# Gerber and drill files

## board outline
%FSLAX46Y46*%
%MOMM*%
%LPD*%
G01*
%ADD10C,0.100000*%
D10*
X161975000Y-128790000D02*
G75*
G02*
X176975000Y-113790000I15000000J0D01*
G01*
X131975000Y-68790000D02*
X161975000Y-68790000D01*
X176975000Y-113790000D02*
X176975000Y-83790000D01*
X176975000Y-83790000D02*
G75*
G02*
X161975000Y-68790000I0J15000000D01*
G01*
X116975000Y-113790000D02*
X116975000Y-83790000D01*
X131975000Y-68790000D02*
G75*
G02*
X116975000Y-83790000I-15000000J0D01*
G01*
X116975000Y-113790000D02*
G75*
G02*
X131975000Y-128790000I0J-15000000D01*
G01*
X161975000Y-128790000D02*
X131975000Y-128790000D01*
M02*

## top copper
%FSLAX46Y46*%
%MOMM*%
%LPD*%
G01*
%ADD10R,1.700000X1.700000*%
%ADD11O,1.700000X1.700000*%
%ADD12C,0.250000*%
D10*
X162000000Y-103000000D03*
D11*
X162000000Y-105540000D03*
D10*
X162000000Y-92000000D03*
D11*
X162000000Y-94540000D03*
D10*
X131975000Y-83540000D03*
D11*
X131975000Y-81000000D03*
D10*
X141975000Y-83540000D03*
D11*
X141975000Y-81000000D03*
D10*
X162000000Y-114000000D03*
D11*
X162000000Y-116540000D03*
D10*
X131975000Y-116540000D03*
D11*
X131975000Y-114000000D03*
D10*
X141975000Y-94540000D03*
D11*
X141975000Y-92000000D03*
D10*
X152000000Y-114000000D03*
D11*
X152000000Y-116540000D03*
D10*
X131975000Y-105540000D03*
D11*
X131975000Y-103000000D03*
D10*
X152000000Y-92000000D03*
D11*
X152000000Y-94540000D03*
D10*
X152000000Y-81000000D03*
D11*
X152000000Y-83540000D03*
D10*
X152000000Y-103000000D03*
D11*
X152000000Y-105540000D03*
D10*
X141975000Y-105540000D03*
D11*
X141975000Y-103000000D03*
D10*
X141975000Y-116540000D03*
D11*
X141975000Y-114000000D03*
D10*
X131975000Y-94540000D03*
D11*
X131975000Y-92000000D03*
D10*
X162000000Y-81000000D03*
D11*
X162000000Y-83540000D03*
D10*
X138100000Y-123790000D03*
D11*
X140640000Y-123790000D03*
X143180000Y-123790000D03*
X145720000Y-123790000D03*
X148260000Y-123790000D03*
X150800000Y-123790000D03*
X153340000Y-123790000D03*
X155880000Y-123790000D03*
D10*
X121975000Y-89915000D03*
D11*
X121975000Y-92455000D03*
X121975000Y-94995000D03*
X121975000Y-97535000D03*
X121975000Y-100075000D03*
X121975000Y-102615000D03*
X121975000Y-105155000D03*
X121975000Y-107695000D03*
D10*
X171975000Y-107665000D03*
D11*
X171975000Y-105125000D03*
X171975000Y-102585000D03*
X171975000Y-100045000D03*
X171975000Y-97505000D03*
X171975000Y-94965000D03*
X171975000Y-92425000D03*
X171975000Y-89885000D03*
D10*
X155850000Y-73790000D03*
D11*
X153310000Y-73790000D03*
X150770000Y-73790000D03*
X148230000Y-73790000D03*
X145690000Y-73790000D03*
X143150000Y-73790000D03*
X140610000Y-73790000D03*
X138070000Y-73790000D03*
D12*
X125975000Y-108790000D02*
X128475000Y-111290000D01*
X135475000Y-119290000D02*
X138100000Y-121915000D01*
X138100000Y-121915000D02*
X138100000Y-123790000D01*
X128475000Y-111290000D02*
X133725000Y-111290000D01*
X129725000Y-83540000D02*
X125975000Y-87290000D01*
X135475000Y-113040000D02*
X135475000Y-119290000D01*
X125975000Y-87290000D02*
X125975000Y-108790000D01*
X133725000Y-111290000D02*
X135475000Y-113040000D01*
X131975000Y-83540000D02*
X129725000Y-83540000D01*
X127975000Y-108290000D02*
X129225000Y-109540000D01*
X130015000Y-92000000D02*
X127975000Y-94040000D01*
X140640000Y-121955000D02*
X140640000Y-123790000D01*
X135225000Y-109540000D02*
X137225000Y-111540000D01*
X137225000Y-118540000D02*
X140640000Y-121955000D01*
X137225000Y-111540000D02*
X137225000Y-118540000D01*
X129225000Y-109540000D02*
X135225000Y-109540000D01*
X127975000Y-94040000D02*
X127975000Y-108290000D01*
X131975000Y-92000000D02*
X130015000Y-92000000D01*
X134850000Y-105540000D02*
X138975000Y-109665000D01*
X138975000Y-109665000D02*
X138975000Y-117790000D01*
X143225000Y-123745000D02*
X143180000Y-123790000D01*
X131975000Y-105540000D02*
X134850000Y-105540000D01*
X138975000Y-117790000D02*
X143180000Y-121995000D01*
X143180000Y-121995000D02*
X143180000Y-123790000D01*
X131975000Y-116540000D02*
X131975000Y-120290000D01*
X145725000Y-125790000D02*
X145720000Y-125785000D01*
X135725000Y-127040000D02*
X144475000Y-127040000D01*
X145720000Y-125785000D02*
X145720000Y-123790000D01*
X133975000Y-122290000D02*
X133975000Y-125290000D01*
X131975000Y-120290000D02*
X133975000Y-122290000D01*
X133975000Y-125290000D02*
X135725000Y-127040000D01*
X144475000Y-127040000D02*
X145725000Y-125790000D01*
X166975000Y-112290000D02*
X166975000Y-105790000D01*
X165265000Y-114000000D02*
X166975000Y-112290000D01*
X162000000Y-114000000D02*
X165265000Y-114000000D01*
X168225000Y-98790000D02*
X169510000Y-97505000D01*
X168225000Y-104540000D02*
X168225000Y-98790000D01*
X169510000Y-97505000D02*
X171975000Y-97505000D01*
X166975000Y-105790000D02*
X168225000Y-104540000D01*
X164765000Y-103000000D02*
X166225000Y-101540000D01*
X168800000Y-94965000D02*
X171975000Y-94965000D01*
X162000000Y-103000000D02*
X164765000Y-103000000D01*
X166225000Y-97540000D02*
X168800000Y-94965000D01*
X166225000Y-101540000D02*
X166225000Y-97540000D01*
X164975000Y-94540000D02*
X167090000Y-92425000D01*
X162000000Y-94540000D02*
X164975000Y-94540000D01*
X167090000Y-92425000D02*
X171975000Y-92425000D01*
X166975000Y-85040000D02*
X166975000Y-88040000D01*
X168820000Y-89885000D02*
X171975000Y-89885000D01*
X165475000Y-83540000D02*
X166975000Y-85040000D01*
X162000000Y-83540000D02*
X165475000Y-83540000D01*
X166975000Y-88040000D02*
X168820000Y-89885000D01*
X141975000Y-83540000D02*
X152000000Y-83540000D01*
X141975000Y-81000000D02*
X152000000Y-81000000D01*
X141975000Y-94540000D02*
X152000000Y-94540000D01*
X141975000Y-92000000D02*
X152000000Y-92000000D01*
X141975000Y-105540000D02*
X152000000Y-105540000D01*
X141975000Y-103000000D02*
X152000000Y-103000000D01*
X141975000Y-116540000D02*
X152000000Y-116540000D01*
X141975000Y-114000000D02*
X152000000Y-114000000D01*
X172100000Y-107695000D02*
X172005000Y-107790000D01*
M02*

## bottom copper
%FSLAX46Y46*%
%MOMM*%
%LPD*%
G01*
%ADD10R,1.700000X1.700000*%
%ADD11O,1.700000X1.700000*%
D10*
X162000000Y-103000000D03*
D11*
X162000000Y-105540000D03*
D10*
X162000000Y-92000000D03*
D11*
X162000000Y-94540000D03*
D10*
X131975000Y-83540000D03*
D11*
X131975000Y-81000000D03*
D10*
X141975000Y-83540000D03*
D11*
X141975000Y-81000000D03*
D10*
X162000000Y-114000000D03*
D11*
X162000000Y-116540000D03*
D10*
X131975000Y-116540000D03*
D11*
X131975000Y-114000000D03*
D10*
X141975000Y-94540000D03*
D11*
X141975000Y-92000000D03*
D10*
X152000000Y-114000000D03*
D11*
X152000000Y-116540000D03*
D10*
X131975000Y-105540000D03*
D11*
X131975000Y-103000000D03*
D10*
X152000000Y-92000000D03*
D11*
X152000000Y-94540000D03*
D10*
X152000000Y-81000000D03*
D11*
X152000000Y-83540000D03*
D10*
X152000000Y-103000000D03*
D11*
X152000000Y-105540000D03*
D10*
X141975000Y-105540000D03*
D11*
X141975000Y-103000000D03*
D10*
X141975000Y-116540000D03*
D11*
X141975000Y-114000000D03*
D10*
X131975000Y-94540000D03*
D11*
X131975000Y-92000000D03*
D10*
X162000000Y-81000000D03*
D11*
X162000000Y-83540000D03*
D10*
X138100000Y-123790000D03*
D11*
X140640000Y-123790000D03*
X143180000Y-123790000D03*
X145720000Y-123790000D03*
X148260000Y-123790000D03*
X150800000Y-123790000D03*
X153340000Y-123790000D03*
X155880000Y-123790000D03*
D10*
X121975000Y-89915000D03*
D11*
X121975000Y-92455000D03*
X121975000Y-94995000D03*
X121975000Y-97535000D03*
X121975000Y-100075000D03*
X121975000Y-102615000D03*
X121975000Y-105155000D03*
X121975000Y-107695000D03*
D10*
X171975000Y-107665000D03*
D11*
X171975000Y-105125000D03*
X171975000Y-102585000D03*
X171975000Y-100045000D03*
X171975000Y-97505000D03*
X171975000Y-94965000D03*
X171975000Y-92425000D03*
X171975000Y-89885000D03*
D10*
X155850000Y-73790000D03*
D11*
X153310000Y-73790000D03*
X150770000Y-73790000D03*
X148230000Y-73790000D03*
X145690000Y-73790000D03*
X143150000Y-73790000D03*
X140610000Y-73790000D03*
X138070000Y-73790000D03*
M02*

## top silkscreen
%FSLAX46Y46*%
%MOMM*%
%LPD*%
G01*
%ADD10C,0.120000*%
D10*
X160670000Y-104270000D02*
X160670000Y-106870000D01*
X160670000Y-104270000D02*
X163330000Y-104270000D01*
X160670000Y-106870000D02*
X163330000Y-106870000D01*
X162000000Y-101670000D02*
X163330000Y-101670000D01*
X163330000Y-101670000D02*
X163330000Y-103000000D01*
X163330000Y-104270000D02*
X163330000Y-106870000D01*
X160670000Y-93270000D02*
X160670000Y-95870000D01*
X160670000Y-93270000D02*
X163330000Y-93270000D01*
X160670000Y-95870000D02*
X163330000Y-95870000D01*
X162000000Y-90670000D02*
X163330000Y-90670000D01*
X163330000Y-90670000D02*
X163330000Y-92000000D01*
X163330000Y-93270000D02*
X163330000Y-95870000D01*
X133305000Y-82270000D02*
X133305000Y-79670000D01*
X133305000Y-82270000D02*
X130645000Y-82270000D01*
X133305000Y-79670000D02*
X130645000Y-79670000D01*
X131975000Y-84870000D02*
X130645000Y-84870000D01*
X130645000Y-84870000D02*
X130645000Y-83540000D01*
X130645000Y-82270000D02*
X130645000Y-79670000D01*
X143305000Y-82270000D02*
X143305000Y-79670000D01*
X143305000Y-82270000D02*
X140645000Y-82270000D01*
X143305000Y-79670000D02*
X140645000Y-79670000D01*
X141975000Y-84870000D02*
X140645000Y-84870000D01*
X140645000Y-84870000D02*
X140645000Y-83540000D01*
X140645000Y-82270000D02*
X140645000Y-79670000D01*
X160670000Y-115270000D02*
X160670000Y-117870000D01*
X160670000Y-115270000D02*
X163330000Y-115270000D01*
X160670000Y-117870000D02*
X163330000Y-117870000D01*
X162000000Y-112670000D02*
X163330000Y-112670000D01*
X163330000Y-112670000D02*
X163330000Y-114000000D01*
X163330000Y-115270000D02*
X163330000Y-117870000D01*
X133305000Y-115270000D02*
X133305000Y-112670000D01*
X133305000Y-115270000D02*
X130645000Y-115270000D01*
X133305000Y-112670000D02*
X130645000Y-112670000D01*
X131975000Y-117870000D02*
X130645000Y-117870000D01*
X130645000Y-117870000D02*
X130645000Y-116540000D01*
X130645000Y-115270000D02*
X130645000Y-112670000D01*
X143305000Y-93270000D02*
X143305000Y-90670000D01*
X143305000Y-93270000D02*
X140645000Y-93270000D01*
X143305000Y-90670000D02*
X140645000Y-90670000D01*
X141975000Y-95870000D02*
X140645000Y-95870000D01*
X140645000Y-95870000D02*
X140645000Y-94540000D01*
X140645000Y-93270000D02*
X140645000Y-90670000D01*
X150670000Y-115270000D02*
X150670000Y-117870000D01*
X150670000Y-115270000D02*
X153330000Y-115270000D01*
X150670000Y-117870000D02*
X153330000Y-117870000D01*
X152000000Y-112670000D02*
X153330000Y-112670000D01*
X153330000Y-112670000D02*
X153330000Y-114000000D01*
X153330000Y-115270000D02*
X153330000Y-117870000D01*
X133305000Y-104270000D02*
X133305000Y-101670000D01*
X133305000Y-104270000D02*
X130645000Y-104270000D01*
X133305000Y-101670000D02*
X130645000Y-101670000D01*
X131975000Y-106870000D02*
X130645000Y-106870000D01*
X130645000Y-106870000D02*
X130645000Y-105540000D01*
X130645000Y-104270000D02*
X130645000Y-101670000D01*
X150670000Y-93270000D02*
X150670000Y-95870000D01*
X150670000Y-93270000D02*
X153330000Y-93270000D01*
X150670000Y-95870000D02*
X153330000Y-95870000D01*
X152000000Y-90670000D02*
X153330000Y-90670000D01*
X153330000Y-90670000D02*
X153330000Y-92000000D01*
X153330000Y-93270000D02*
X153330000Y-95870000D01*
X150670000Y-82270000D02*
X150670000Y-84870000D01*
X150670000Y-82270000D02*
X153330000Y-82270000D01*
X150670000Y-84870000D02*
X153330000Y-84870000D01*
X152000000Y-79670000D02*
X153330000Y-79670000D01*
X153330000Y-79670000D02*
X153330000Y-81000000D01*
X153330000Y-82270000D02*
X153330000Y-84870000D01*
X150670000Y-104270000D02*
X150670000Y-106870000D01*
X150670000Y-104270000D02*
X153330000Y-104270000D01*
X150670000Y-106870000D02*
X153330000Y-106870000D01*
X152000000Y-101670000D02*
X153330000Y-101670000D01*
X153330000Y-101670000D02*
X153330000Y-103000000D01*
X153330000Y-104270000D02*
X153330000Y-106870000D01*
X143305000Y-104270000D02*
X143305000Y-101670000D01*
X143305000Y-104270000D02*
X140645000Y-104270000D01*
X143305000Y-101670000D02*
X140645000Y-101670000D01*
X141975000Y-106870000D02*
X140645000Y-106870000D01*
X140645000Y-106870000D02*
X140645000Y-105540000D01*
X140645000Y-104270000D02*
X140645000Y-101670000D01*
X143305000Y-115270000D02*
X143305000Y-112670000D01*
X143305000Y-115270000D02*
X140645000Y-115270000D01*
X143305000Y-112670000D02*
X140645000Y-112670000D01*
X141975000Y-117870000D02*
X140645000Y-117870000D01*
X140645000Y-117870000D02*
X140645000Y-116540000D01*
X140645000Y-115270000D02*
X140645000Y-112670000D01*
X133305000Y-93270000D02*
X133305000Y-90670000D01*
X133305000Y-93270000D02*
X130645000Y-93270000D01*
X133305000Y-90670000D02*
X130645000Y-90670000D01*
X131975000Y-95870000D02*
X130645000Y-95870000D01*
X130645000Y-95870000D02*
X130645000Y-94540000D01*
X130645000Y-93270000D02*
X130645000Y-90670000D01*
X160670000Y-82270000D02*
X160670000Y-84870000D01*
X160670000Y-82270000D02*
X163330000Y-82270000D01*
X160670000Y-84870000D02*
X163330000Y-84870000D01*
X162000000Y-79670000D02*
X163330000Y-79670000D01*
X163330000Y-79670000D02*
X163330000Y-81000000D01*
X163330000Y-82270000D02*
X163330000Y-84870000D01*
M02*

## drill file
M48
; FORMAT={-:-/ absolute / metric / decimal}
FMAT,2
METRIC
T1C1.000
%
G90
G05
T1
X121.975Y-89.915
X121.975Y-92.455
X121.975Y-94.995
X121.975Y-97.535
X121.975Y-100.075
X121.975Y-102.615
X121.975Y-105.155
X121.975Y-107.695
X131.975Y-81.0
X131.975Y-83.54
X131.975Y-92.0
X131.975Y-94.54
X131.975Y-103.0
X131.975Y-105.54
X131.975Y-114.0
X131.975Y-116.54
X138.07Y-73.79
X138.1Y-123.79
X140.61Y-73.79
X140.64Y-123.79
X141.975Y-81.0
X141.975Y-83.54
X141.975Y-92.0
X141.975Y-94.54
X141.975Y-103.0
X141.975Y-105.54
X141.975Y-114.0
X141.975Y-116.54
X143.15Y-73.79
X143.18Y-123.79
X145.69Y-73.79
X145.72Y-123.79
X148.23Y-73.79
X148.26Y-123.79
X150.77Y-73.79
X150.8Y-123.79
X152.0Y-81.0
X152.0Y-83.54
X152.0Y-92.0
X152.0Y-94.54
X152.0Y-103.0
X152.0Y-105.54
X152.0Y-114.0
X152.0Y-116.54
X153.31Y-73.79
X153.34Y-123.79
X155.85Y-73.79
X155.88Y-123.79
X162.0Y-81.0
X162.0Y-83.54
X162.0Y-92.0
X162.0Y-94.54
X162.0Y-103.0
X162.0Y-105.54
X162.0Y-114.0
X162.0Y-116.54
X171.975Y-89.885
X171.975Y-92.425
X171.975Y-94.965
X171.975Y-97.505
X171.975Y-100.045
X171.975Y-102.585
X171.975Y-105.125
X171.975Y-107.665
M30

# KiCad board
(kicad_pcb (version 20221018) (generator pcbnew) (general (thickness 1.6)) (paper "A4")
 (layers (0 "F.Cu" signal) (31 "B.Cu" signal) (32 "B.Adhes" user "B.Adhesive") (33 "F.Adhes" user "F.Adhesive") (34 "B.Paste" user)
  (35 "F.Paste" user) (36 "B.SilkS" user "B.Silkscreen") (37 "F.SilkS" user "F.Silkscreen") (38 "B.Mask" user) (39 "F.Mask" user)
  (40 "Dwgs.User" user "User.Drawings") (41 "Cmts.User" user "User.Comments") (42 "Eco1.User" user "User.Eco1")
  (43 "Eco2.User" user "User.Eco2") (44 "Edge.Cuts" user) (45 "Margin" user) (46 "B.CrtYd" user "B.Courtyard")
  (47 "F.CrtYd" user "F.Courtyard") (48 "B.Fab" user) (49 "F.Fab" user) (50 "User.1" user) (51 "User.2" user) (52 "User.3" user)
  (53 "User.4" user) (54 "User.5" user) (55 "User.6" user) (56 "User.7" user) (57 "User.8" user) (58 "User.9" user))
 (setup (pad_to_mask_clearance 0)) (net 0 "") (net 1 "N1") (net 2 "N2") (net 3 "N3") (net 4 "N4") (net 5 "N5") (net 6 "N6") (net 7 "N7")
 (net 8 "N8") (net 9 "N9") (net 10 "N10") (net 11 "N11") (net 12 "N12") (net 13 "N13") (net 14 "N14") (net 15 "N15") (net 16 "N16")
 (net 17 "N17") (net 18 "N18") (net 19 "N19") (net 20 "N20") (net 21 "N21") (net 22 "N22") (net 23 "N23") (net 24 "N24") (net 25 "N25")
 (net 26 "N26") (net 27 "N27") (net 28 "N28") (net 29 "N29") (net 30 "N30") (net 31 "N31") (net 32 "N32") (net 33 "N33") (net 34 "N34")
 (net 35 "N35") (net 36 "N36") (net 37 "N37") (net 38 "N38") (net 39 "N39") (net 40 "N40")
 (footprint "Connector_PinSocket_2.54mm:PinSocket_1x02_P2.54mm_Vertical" (layer "F.Cu") (at 162 103)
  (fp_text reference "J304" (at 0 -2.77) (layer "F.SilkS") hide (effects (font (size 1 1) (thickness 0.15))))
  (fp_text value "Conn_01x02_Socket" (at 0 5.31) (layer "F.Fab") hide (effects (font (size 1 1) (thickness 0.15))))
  (fp_line (start -1.33 1.27) (end -1.33 3.87) (stroke (width 0.12) (type solid)) (layer "F.SilkS"))
  (fp_line (start -1.33 1.27) (end 1.33 1.27) (stroke (width 0.12) (type solid)) (layer "F.SilkS"))
  (fp_line (start -1.33 3.87) (end 1.33 3.87) (stroke (width 0.12) (type solid)) (layer "F.SilkS"))
  (fp_line (start 0 -1.33) (end 1.33 -1.33) (stroke (width 0.12) (type solid)) (layer "F.SilkS"))
  (fp_line (start 1.33 -1.33) (end 1.33 0) (stroke (width 0.12) (type solid)) (layer "F.SilkS"))
  (fp_line (start 1.33 1.27) (end 1.33 3.87) (stroke (width 0.12) (type solid)) (layer "F.SilkS"))
  (pad "1" thru_hole rect (at 0 0) (size 1.7 1.7) (drill 1) (layers "*.Cu" "*.Mask") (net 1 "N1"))
  (pad "2" thru_hole oval (at 0 2.54) (size 1.7 1.7) (drill 1) (layers "*.Cu" "*.Mask") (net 1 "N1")))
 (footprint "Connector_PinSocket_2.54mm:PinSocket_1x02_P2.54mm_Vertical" (layer "F.Cu") (at 162 92)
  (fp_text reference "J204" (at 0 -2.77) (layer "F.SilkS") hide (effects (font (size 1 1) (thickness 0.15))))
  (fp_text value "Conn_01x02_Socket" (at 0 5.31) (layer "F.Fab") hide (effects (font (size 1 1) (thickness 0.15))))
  (fp_line (start -1.33 1.27) (end -1.33 3.87) (stroke (width 0.12) (type solid)) (layer "F.SilkS"))
  (fp_line (start -1.33 1.27) (end 1.33 1.27) (stroke (width 0.12) (type solid)) (layer "F.SilkS"))
  (fp_line (start -1.33 3.87) (end 1.33 3.87) (stroke (width 0.12) (type solid)) (layer "F.SilkS"))
  (fp_line (start 0 -1.33) (end 1.33 -1.33) (stroke (width 0.12) (type solid)) (layer "F.SilkS"))
  (fp_line (start 1.33 -1.33) (end 1.33 0) (stroke (width 0.12) (type solid)) (layer "F.SilkS"))
  (fp_line (start 1.33 1.27) (end 1.33 3.87) (stroke (width 0.12) (type solid)) (layer "F.SilkS"))
  (pad "1" thru_hole rect (at 0 0) (size 1.7 1.7) (drill 1) (layers "*.Cu" "*.Mask") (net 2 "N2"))
  (pad "2" thru_hole oval (at 0 2.54) (size 1.7 1.7) (drill 1) (layers "*.Cu" "*.Mask") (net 2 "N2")))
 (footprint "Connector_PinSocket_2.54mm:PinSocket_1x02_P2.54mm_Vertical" (layer "F.Cu") (at 131.975 83.54 180)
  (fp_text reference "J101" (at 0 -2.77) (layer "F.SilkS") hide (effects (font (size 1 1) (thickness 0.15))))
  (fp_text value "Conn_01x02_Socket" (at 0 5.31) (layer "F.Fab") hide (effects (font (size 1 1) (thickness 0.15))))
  (fp_line (start -1.33 1.27) (end -1.33 3.87) (stroke (width 0.12) (type solid)) (layer "F.SilkS"))
  (fp_line (start -1.33 1.27) (end 1.33 1.27) (stroke (width 0.12) (type solid)) (layer "F.SilkS"))
  (fp_line (start -1.33 3.87) (end 1.33 3.87) (stroke (width 0.12) (type solid)) (layer "F.SilkS"))
  (fp_line (start 0 -1.33) (end 1.33 -1.33) (stroke (width 0.12) (type solid)) (layer "F.SilkS"))
  (fp_line (start 1.33 -1.33) (end 1.33 0) (stroke (width 0.12) (type solid)) (layer "F.SilkS"))
  (fp_line (start 1.33 1.27) (end 1.33 3.87) (stroke (width 0.12) (type solid)) (layer "F.SilkS"))
  (pad "1" thru_hole rect (at 0 0 180) (size 1.7 1.7) (drill 1) (layers "*.Cu" "*.Mask") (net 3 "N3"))
  (pad "2" thru_hole oval (at 0 2.54 180) (size 1.7 1.7) (drill 1) (layers "*.Cu" "*.Mask") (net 3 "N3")))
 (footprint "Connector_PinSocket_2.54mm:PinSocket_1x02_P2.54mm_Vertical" (layer "F.Cu") (at 141.975 83.54 180)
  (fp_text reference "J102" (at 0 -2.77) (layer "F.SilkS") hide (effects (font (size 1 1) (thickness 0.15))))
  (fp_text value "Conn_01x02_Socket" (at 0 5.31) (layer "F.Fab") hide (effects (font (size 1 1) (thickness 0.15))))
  (fp_line (start -1.33 1.27) (end -1.33 3.87) (stroke (width 0.12) (type solid)) (layer "F.SilkS"))
  (fp_line (start -1.33 1.27) (end 1.33 1.27) (stroke (width 0.12) (type solid)) (layer "F.SilkS"))
  (fp_line (start -1.33 3.87) (end 1.33 3.87) (stroke (width 0.12) (type solid)) (layer "F.SilkS"))
  (fp_line (start 0 -1.33) (end 1.33 -1.33) (stroke (width 0.12) (type solid)) (layer "F.SilkS"))
  (fp_line (start 1.33 -1.33) (end 1.33 0) (stroke (width 0.12) (type solid)) (layer "F.SilkS"))
  (fp_line (start 1.33 1.27) (end 1.33 3.87) (stroke (width 0.12) (type solid)) (layer "F.SilkS"))
  (pad "1" thru_hole rect (at 0 0 180) (size 1.7 1.7) (drill 1) (layers "*.Cu" "*.Mask") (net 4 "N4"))
  (pad "2" thru_hole oval (at 0 2.54 180) (size 1.7 1.7) (drill 1) (layers "*.Cu" "*.Mask") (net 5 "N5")))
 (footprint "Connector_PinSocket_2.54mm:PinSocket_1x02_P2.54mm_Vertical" (layer "F.Cu") (at 162 114)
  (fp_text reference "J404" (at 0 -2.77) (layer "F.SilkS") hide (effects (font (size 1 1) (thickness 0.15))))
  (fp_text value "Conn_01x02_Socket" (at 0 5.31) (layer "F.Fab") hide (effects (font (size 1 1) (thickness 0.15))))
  (fp_line (start -1.33 1.27) (end -1.33 3.87) (stroke (width 0.12) (type solid)) (layer "F.SilkS"))
  (fp_line (start -1.33 1.27) (end 1.33 1.27) (stroke (width 0.12) (type solid)) (layer "F.SilkS"))
  (fp_line (start -1.33 3.87) (end 1.33 3.87) (stroke (width 0.12) (type solid)) (layer "F.SilkS"))
  (fp_line (start 0 -1.33) (end 1.33 -1.33) (stroke (width 0.12) (type solid)) (layer "F.SilkS"))
  (fp_line (start 1.33 -1.33) (end 1.33 0) (stroke (width 0.12) (type solid)) (layer "F.SilkS"))
  (fp_line (start 1.33 1.27) (end 1.33 3.87) (stroke (width 0.12) (type solid)) (layer "F.SilkS"))
  (pad "1" thru_hole rect (at 0 0) (size 1.7 1.7) (drill 1) (layers "*.Cu" "*.Mask") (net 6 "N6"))
  (pad "2" thru_hole oval (at 0 2.54) (size 1.7 1.7) (drill 1) (layers "*.Cu" "*.Mask") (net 6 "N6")))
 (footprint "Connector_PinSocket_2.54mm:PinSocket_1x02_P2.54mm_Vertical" (layer "F.Cu") (at 131.975 116.54 180)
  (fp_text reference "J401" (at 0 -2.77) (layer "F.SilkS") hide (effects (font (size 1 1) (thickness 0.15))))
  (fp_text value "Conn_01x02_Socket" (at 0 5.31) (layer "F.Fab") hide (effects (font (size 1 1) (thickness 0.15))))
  (fp_line (start -1.33 1.27) (end -1.33 3.87) (stroke (width 0.12) (type solid)) (layer "F.SilkS"))
  (fp_line (start -1.33 1.27) (end 1.33 1.27) (stroke (width 0.12) (type solid)) (layer "F.SilkS"))
  (fp_line (start -1.33 3.87) (end 1.33 3.87) (stroke (width 0.12) (type solid)) (layer "F.SilkS"))
  (fp_line (start 0 -1.33) (end 1.33 -1.33) (stroke (width 0.12) (type solid)) (layer "F.SilkS"))
  (fp_line (start 1.33 -1.33) (end 1.33 0) (stroke (width 0.12) (type solid)) (layer "F.SilkS"))
  (fp_line (start 1.33 1.27) (end 1.33 3.87) (stroke (width 0.12) (type solid)) (layer "F.SilkS"))
  (pad "1" thru_hole rect (at 0 0 180) (size 1.7 1.7) (drill 1) (layers "*.Cu" "*.Mask") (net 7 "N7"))
  (pad "2" thru_hole oval (at 0 2.54 180) (size 1.7 1.7) (drill 1) (layers "*.Cu" "*.Mask") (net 7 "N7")))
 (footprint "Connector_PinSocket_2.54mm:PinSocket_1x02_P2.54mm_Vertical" (layer "F.Cu") (at 141.975 94.54 180)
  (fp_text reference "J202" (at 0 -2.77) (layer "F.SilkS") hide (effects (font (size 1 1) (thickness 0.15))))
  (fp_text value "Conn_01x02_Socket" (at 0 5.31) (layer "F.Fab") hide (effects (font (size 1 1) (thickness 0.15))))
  (fp_line (start -1.33 1.27) (end -1.33 3.87) (stroke (width 0.12) (type solid)) (layer "F.SilkS"))
  (fp_line (start -1.33 1.27) (end 1.33 1.27) (stroke (width 0.12) (type solid)) (layer "F.SilkS"))
  (fp_line (start -1.33 3.87) (end 1.33 3.87) (stroke (width 0.12) (type solid)) (layer "F.SilkS"))
  (fp_line (start 0 -1.33) (end 1.33 -1.33) (stroke (width 0.12) (type solid)) (layer "F.SilkS"))
  (fp_line (start 1.33 -1.33) (end 1.33 0) (stroke (width 0.12) (type solid)) (layer "F.SilkS"))
  (fp_line (start 1.33 1.27) (end 1.33 3.87) (stroke (width 0.12) (type solid)) (layer "F.SilkS"))
  (pad "1" thru_hole rect (at 0 0 180) (size 1.7 1.7) (drill 1) (layers "*.Cu" "*.Mask") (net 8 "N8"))
  (pad "2" thru_hole oval (at 0 2.54 180) (size 1.7 1.7) (drill 1) (layers "*.Cu" "*.Mask") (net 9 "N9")))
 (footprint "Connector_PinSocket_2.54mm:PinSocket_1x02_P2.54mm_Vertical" (layer "F.Cu") (at 152 114)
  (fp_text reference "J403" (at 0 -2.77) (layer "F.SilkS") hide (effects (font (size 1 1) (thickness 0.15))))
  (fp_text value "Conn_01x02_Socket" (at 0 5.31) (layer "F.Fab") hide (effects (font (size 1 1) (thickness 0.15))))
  (fp_line (start -1.33 1.27) (end -1.33 3.87) (stroke (width 0.12) (type solid)) (layer "F.SilkS"))
  (fp_line (start -1.33 1.27) (end 1.33 1.27) (stroke (width 0.12) (type solid)) (layer "F.SilkS"))
  (fp_line (start -1.33 3.87) (end 1.33 3.87) (stroke (width 0.12) (type solid)) (layer "F.SilkS"))
  (fp_line (start 0 -1.33) (end 1.33 -1.33) (stroke (width 0.12) (type solid)) (layer "F.SilkS"))
  (fp_line (start 1.33 -1.33) (end 1.33 0) (stroke (width 0.12) (type solid)) (layer "F.SilkS"))
  (fp_line (start 1.33 1.27) (end 1.33 3.87) (stroke (width 0.12) (type solid)) (layer "F.SilkS"))
  (pad "1" thru_hole rect (at 0 0) (size 1.7 1.7) (drill 1) (layers "*.Cu" "*.Mask") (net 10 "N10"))
  (pad "2" thru_hole oval (at 0 2.54) (size 1.7 1.7) (drill 1) (layers "*.Cu" "*.Mask") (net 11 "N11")))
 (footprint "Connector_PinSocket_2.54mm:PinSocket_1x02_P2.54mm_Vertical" (layer "F.Cu") (at 131.975 105.54 180)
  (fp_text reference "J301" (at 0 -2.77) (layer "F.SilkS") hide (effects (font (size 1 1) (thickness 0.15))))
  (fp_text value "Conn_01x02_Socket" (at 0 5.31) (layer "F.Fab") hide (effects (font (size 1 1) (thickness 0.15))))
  (fp_line (start -1.33 1.27) (end -1.33 3.87) (stroke (width 0.12) (type solid)) (layer "F.SilkS"))
  (fp_line (start -1.33 1.27) (end 1.33 1.27) (stroke (width 0.12) (type solid)) (layer "F.SilkS"))
  (fp_line (start -1.33 3.87) (end 1.33 3.87) (stroke (width 0.12) (type solid)) (layer "F.SilkS"))
  (fp_line (start 0 -1.33) (end 1.33 -1.33) (stroke (width 0.12) (type solid)) (layer "F.SilkS"))
  (fp_line (start 1.33 -1.33) (end 1.33 0) (stroke (width 0.12) (type solid)) (layer "F.SilkS"))
  (fp_line (start 1.33 1.27) (end 1.33 3.87) (stroke (width 0.12) (type solid)) (layer "F.SilkS"))
  (pad "1" thru_hole rect (at 0 0 180) (size 1.7 1.7) (drill 1) (layers "*.Cu" "*.Mask") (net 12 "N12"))
  (pad "2" thru_hole oval (at 0 2.54 180) (size 1.7 1.7) (drill 1) (layers "*.Cu" "*.Mask") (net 12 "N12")))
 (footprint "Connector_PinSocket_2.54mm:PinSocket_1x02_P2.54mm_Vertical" (layer "F.Cu") (at 152 92)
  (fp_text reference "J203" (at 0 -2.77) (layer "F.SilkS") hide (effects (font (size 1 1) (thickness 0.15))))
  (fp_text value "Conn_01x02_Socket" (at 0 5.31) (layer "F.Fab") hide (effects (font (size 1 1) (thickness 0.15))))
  (fp_line (start -1.33 1.27) (end -1.33 3.87) (stroke (width 0.12) (type solid)) (layer "F.SilkS"))
  (fp_line (start -1.33 1.27) (end 1.33 1.27) (stroke (width 0.12) (type solid)) (layer "F.SilkS"))
  (fp_line (start -1.33 3.87) (end 1.33 3.87) (stroke (width 0.12) (type solid)) (layer "F.SilkS"))
  (fp_line (start 0 -1.33) (end 1.33 -1.33) (stroke (width 0.12) (type solid)) (layer "F.SilkS"))
  (fp_line (start 1.33 -1.33) (end 1.33 0) (stroke (width 0.12) (type solid)) (layer "F.SilkS"))
  (fp_line (start 1.33 1.27) (end 1.33 3.87) (stroke (width 0.12) (type solid)) (layer "F.SilkS"))
  (pad "1" thru_hole rect (at 0 0) (size 1.7 1.7) (drill 1) (layers "*.Cu" "*.Mask") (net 9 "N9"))
  (pad "2" thru_hole oval (at 0 2.54) (size 1.7 1.7) (drill 1) (layers "*.Cu" "*.Mask") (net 8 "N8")))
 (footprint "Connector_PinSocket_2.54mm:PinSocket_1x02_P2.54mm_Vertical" (layer "F.Cu") (at 152 81)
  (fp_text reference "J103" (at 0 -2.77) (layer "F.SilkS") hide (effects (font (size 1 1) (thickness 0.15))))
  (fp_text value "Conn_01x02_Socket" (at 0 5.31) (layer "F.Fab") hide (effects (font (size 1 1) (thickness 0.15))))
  (fp_line (start -1.33 1.27) (end -1.33 3.87) (stroke (width 0.12) (type solid)) (layer "F.SilkS"))
  (fp_line (start -1.33 1.27) (end 1.33 1.27) (stroke (width 0.12) (type solid)) (layer "F.SilkS"))
  (fp_line (start -1.33 3.87) (end 1.33 3.87) (stroke (width 0.12) (type solid)) (layer "F.SilkS"))
  (fp_line (start 0 -1.33) (end 1.33 -1.33) (stroke (width 0.12) (type solid)) (layer "F.SilkS"))
  (fp_line (start 1.33 -1.33) (end 1.33 0) (stroke (width 0.12) (type solid)) (layer "F.SilkS"))
  (fp_line (start 1.33 1.27) (end 1.33 3.87) (stroke (width 0.12) (type solid)) (layer "F.SilkS"))
  (pad "1" thru_hole rect (at 0 0) (size 1.7 1.7) (drill 1) (layers "*.Cu" "*.Mask") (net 5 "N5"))
  (pad "2" thru_hole oval (at 0 2.54) (size 1.7 1.7) (drill 1) (layers "*.Cu" "*.Mask") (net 4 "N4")))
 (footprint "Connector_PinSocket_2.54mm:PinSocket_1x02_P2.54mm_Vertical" (layer "F.Cu") (at 152 103)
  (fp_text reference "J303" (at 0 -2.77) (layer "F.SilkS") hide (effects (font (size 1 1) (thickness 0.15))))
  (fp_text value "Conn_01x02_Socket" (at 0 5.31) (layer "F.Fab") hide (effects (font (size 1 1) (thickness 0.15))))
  (fp_line (start -1.33 1.27) (end -1.33 3.87) (stroke (width 0.12) (type solid)) (layer "F.SilkS"))
  (fp_line (start -1.33 1.27) (end 1.33 1.27) (stroke (width 0.12) (type solid)) (layer "F.SilkS"))
  (fp_line (start -1.33 3.87) (end 1.33 3.87) (stroke (width 0.12) (type solid)) (layer "F.SilkS"))
  (fp_line (start 0 -1.33) (end 1.33 -1.33) (stroke (width 0.12) (type solid)) (layer "F.SilkS"))
  (fp_line (start 1.33 -1.33) (end 1.33 0) (stroke (width 0.12) (type solid)) (layer "F.SilkS"))
  (fp_line (start 1.33 1.27) (end 1.33 3.87) (stroke (width 0.12) (type solid)) (layer "F.SilkS"))
  (pad "1" thru_hole rect (at 0 0) (size 1.7 1.7) (drill 1) (layers "*.Cu" "*.Mask") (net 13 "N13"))
  (pad "2" thru_hole oval (at 0 2.54) (size 1.7 1.7) (drill 1) (layers "*.Cu" "*.Mask") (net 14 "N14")))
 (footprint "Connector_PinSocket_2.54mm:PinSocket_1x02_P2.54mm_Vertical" (layer "F.Cu") (at 141.975 105.54 180)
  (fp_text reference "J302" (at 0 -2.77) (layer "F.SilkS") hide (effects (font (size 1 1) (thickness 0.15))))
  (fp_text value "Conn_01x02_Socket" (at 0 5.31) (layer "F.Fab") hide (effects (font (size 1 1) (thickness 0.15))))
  (fp_line (start -1.33 1.27) (end -1.33 3.87) (stroke (width 0.12) (type solid)) (layer "F.SilkS"))
  (fp_line (start -1.33 1.27) (end 1.33 1.27) (stroke (width 0.12) (type solid)) (layer "F.SilkS"))
  (fp_line (start -1.33 3.87) (end 1.33 3.87) (stroke (width 0.12) (type solid)) (layer "F.SilkS"))
  (fp_line (start 0 -1.33) (end 1.33 -1.33) (stroke (width 0.12) (type solid)) (layer "F.SilkS"))
  (fp_line (start 1.33 -1.33) (end 1.33 0) (stroke (width 0.12) (type solid)) (layer "F.SilkS"))
  (fp_line (start 1.33 1.27) (end 1.33 3.87) (stroke (width 0.12) (type solid)) (layer "F.SilkS"))
  (pad "1" thru_hole rect (at 0 0 180) (size 1.7 1.7) (drill 1) (layers "*.Cu" "*.Mask") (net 14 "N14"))
  (pad "2" thru_hole oval (at 0 2.54 180) (size 1.7 1.7) (drill 1) (layers "*.Cu" "*.Mask") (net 13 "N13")))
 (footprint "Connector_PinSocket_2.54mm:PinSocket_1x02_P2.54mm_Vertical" (layer "F.Cu") (at 141.975 116.54 180)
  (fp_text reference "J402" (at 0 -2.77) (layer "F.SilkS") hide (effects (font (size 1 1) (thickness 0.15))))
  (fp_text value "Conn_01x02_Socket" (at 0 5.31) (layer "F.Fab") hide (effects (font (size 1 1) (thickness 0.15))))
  (fp_line (start -1.33 1.27) (end -1.33 3.87) (stroke (width 0.12) (type solid)) (layer "F.SilkS"))
  (fp_line (start -1.33 1.27) (end 1.33 1.27) (stroke (width 0.12) (type solid)) (layer "F.SilkS"))
  (fp_line (start -1.33 3.87) (end 1.33 3.87) (stroke (width 0.12) (type solid)) (layer "F.SilkS"))
  (fp_line (start 0 -1.33) (end 1.33 -1.33) (stroke (width 0.12) (type solid)) (layer "F.SilkS"))
  (fp_line (start 1.33 -1.33) (end 1.33 0) (stroke (width 0.12) (type solid)) (layer "F.SilkS"))
  (fp_line (start 1.33 1.27) (end 1.33 3.87) (stroke (width 0.12) (type solid)) (layer "F.SilkS"))
  (pad "1" thru_hole rect (at 0 0 180) (size 1.7 1.7) (drill 1) (layers "*.Cu" "*.Mask") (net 11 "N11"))
  (pad "2" thru_hole oval (at 0 2.54 180) (size 1.7 1.7) (drill 1) (layers "*.Cu" "*.Mask") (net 10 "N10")))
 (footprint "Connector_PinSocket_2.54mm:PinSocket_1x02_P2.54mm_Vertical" (layer "F.Cu") (at 131.975 94.54 180)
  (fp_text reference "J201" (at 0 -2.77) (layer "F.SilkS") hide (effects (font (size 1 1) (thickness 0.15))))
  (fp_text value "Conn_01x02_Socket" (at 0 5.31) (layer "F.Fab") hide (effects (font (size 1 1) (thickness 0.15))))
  (fp_line (start -1.33 1.27) (end -1.33 3.87) (stroke (width 0.12) (type solid)) (layer "F.SilkS"))
  (fp_line (start -1.33 1.27) (end 1.33 1.27) (stroke (width 0.12) (type solid)) (layer "F.SilkS"))
  (fp_line (start -1.33 3.87) (end 1.33 3.87) (stroke (width 0.12) (type solid)) (layer "F.SilkS"))
  (fp_line (start 0 -1.33) (end 1.33 -1.33) (stroke (width 0.12) (type solid)) (layer "F.SilkS"))
  (fp_line (start 1.33 -1.33) (end 1.33 0) (stroke (width 0.12) (type solid)) (layer "F.SilkS"))
  (fp_line (start 1.33 1.27) (end 1.33 3.87) (stroke (width 0.12) (type solid)) (layer "F.SilkS"))
  (pad "1" thru_hole rect (at 0 0 180) (size 1.7 1.7) (drill 1) (layers "*.Cu" "*.Mask") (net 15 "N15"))
  (pad "2" thru_hole oval (at 0 2.54 180) (size 1.7 1.7) (drill 1) (layers "*.Cu" "*.Mask") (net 15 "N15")))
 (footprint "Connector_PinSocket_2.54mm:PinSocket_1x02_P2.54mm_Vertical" (layer "F.Cu") (at 162 81)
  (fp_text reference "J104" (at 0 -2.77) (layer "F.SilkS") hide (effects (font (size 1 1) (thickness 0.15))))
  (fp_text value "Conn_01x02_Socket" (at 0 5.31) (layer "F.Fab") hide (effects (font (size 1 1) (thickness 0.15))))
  (fp_line (start -1.33 1.27) (end -1.33 3.87) (stroke (width 0.12) (type solid)) (layer "F.SilkS"))
  (fp_line (start -1.33 1.27) (end 1.33 1.27) (stroke (width 0.12) (type solid)) (layer "F.SilkS"))
  (fp_line (start -1.33 3.87) (end 1.33 3.87) (stroke (width 0.12) (type solid)) (layer "F.SilkS"))
  (fp_line (start 0 -1.33) (end 1.33 -1.33) (stroke (width 0.12) (type solid)) (layer "F.SilkS"))
  (fp_line (start 1.33 -1.33) (end 1.33 0) (stroke (width 0.12) (type solid)) (layer "F.SilkS"))
  (fp_line (start 1.33 1.27) (end 1.33 3.87) (stroke (width 0.12) (type solid)) (layer "F.SilkS"))
  (pad "1" thru_hole rect (at 0 0) (size 1.7 1.7) (drill 1) (layers "*.Cu" "*.Mask") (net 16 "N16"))
  (pad "2" thru_hole oval (at 0 2.54) (size 1.7 1.7) (drill 1) (layers "*.Cu" "*.Mask") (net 16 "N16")))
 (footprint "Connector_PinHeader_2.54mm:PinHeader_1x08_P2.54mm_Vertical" (layer "B.Cu") (at 138.1 123.79 -90)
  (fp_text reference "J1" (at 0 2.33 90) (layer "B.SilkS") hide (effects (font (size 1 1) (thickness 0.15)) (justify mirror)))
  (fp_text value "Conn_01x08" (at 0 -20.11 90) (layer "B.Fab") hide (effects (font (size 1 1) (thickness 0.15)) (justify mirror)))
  (pad "1" thru_hole rect (at 0 0 270) (size 1.7 1.7) (drill 1) (layers "*.Cu" "*.Mask") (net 3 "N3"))
  (pad "2" thru_hole oval (at 0 -2.54 270) (size 1.7 1.7) (drill 1) (layers "*.Cu" "*.Mask") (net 15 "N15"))
  (pad "3" thru_hole oval (at 0 -5.08 270) (size 1.7 1.7) (drill 1) (layers "*.Cu" "*.Mask") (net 12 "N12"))
  (pad "4" thru_hole oval (at 0 -7.62 270) (size 1.7 1.7) (drill 1) (layers "*.Cu" "*.Mask") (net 7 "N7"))
  (pad "5" thru_hole oval (at 0 -10.16 270) (size 1.7 1.7) (drill 1) (layers "*.Cu" "*.Mask") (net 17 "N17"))
  (pad "6" thru_hole oval (at 0 -12.7 270) (size 1.7 1.7) (drill 1) (layers "*.Cu" "*.Mask") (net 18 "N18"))
  (pad "7" thru_hole oval (at 0 -15.24 270) (size 1.7 1.7) (drill 1) (layers "*.Cu" "*.Mask") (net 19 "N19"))
  (pad "8" thru_hole oval (at 0 -17.78 270) (size 1.7 1.7) (drill 1) (layers "*.Cu" "*.Mask") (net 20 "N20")))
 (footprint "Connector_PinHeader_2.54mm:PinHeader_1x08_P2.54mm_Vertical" (layer "B.Cu") (at 121.975 89.915 180)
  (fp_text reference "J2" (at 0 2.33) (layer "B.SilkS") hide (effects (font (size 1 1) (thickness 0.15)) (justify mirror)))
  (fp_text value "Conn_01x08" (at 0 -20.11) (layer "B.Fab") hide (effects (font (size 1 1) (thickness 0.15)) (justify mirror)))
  (pad "1" thru_hole rect (at 0 0 180) (size 1.7 1.7) (drill 1) (layers "*.Cu" "*.Mask") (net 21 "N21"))
  (pad "2" thru_hole oval (at 0 -2.54 180) (size 1.7 1.7) (drill 1) (layers "*.Cu" "*.Mask") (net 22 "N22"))
  (pad "3" thru_hole oval (at 0 -5.08 180) (size 1.7 1.7) (drill 1) (layers "*.Cu" "*.Mask") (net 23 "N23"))
  (pad "4" thru_hole oval (at 0 -7.62 180) (size 1.7 1.7) (drill 1) (layers "*.Cu" "*.Mask") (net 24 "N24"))
  (pad "5" thru_hole oval (at 0 -10.16 180) (size 1.7 1.7) (drill 1) (layers "*.Cu" "*.Mask") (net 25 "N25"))
  (pad "6" thru_hole oval (at 0 -12.7 180) (size 1.7 1.7) (drill 1) (layers "*.Cu" "*.Mask") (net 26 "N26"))
  (pad "7" thru_hole oval (at 0 -15.24 180) (size 1.7 1.7) (drill 1) (layers "*.Cu" "*.Mask") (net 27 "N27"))
  (pad "8" thru_hole oval (at 0 -17.78 180) (size 1.7 1.7) (drill 1) (layers "*.Cu" "*.Mask") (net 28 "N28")))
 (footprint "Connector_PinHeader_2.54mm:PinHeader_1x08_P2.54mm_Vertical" (layer "B.Cu") (at 171.975 107.665)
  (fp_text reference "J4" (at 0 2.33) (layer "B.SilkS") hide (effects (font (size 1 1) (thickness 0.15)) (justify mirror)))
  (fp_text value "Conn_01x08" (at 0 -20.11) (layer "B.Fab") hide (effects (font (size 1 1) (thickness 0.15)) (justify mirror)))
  (pad "1" thru_hole rect (at 0 0) (size 1.7 1.7) (drill 1) (layers "*.Cu" "*.Mask") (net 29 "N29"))
  (pad "2" thru_hole oval (at 0 -2.54) (size 1.7 1.7) (drill 1) (layers "*.Cu" "*.Mask") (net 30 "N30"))
  (pad "3" thru_hole oval (at 0 -5.08) (size 1.7 1.7) (drill 1) (layers "*.Cu" "*.Mask") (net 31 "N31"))
  (pad "4" thru_hole oval (at 0 -7.62) (size 1.7 1.7) (drill 1) (layers "*.Cu" "*.Mask") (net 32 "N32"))
  (pad "5" thru_hole oval (at 0 -10.16) (size 1.7 1.7) (drill 1) (layers "*.Cu" "*.Mask") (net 6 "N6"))
  (pad "6" thru_hole oval (at 0 -12.7) (size 1.7 1.7) (drill 1) (layers "*.Cu" "*.Mask") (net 1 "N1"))
  (pad "7" thru_hole oval (at 0 -15.24) (size 1.7 1.7) (drill 1) (layers "*.Cu" "*.Mask") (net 2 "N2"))
  (pad "8" thru_hole oval (at 0 -17.78) (size 1.7 1.7) (drill 1) (layers "*.Cu" "*.Mask") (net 16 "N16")))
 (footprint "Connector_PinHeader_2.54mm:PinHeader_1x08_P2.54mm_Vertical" (layer "B.Cu") (at 155.85 73.79 90)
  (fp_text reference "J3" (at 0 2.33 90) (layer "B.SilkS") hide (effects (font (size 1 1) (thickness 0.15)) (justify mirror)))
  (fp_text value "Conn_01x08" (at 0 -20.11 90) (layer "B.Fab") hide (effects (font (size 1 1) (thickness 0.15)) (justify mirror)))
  (pad "1" thru_hole rect (at 0 0 90) (size 1.7 1.7) (drill 1) (layers "*.Cu" "*.Mask") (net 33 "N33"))
  (pad "2" thru_hole oval (at 0 -2.54 90) (size 1.7 1.7) (drill 1) (layers "*.Cu" "*.Mask") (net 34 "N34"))
  (pad "3" thru_hole oval (at 0 -5.08 90) (size 1.7 1.7) (drill 1) (layers "*.Cu" "*.Mask") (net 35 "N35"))
  (pad "4" thru_hole oval (at 0 -7.62 90) (size 1.7 1.7) (drill 1) (layers "*.Cu" "*.Mask") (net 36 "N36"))
  (pad "5" thru_hole oval (at 0 -10.16 90) (size 1.7 1.7) (drill 1) (layers "*.Cu" "*.Mask") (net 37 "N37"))
  (pad "6" thru_hole oval (at 0 -12.7 90) (size 1.7 1.7) (drill 1) (layers "*.Cu" "*.Mask") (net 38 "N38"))
  (pad "7" thru_hole oval (at 0 -15.24 90) (size 1.7 1.7) (drill 1) (layers "*.Cu" "*.Mask") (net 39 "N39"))
  (pad "8" thru_hole oval (at 0 -17.78 90) (size 1.7 1.7) (drill 1) (layers "*.Cu" "*.Mask") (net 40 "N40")))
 (gr_arc (start 161.975 128.79) (mid 166.368398 118.183398) (end 176.975 113.79) (stroke (width 0.1) (type default)) (layer "Edge.Cuts"))
 (gr_line (start 131.975 68.79) (end 161.975 68.79) (stroke (width 0.1) (type default)) (layer "Edge.Cuts"))
 (gr_line (start 176.975 113.79) (end 176.975 83.79) (stroke (width 0.1) (type default)) (layer "Edge.Cuts"))
 (gr_arc (start 176.975 83.79) (mid 166.368398 79.396602) (end 161.975 68.79) (stroke (width 0.1) (type default)) (layer "Edge.Cuts"))
 (gr_line (start 116.975 113.79) (end 116.975 83.79) (stroke (width 0.1) (type default)) (layer "Edge.Cuts"))
 (gr_arc (start 131.975 68.79) (mid 127.581602 79.396602) (end 116.975 83.79) (stroke (width 0.1) (type default)) (layer "Edge.Cuts"))
 (gr_arc (start 116.975 113.79) (mid 127.581602 118.183398) (end 131.975 128.79) (stroke (width 0.1) (type default)) (layer "Edge.Cuts"))
 (gr_line (start 161.975 128.79) (end 131.975 128.79) (stroke (width 0.1) (type default)) (layer "Edge.Cuts"))
 (segment (start 125.975 108.79) (end 128.475 111.29) (width 0.25) (layer "F.Cu") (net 3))
 (segment (start 135.475 119.29) (end 138.1 121.915) (width 0.25) (layer "F.Cu") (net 3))
 (segment (start 138.1 121.915) (end 138.1 123.79) (width 0.25) (layer "F.Cu") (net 3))
 (segment (start 128.475 111.29) (end 133.725 111.29) (width 0.25) (layer "F.Cu") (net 3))
 (segment (start 129.725 83.54) (end 125.975 87.29) (width 0.25) (layer "F.Cu") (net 3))
 (segment (start 135.475 113.04) (end 135.475 119.29) (width 0.25) (layer "F.Cu") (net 3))
 (segment (start 125.975 87.29) (end 125.975 108.79) (width 0.25) (layer "F.Cu") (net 3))
 (segment (start 133.725 111.29) (end 135.475 113.04) (width 0.25) (layer "F.Cu") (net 3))
 (segment (start 131.975 83.54) (end 129.725 83.54) (width 0.25) (layer "F.Cu") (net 3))
 (segment (start 127.975 108.29) (end 129.225 109.54) (width 0.25) (layer "F.Cu") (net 15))
 (segment (start 130.015 92) (end 127.975 94.04) (width 0.25) (layer "F.Cu") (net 15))
 (segment (start 140.64 121.955) (end 140.64 123.79) (width 0.25) (layer "F.Cu") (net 15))
 (segment (start 135.225 109.54) (end 137.225 111.54) (width 0.25) (layer "F.Cu") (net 15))
 (segment (start 137.225 118.54) (end 140.64 121.955) (width 0.25) (layer "F.Cu") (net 15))
 (segment (start 137.225 111.54) (end 137.225 118.54) (width 0.25) (layer "F.Cu") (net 15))
 (segment (start 129.225 109.54) (end 135.225 109.54) (width 0.25) (layer "F.Cu") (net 15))
 (segment (start 127.975 94.04) (end 127.975 108.29) (width 0.25) (layer "F.Cu") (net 15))
 (segment (start 131.975 92) (end 130.015 92) (width 0.25) (layer "F.Cu") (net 15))
 (segment (start 134.85 105.54) (end 138.975 109.665) (width 0.25) (layer "F.Cu") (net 12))
 (segment (start 138.975 109.665) (end 138.975 117.79) (width 0.25) (layer "F.Cu") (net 12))
 (segment (start 143.225 123.745) (end 143.18 123.79) (width 0.25) (layer "F.Cu") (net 12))
 (segment (start 131.975 105.54) (end 134.85 105.54) (width 0.25) (layer "F.Cu") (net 12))
 (segment (start 138.975 117.79) (end 143.18 121.995) (width 0.25) (layer "F.Cu") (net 12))
 (segment (start 143.18 121.995) (end 143.18 123.79) (width 0.25) (layer "F.Cu") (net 12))
 (segment (start 131.975 116.54) (end 131.975 120.29) (width 0.25) (layer "F.Cu") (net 7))
 (segment (start 145.725 125.79) (end 145.72 125.785) (width 0.25) (layer "F.Cu") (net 7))
 (segment (start 135.725 127.04) (end 144.475 127.04) (width 0.25) (layer "F.Cu") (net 7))
 (segment (start 145.72 125.785) (end 145.72 123.79) (width 0.25) (layer "F.Cu") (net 7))
 (segment (start 133.975 122.29) (end 133.975 125.29) (width 0.25) (layer "F.Cu") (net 7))
 (segment (start 131.975 120.29) (end 133.975 122.29) (width 0.25) (layer "F.Cu") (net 7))
 (segment (start 133.975 125.29) (end 135.725 127.04) (width 0.25) (layer "F.Cu") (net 7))
 (segment (start 144.475 127.04) (end 145.725 125.79) (width 0.25) (layer "F.Cu") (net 7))
 (segment (start 166.975 112.29) (end 166.975 105.79) (width 0.25) (layer "F.Cu") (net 6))
 (segment (start 165.265 114) (end 166.975 112.29) (width 0.25) (layer "F.Cu") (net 6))
 (segment (start 162 114) (end 165.265 114) (width 0.25) (layer "F.Cu") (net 6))
 (segment (start 168.225 98.79) (end 169.51 97.505) (width 0.25) (layer "F.Cu") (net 6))
 (segment (start 168.225 104.54) (end 168.225 98.79) (width 0.25) (layer "F.Cu") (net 6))
 (segment (start 169.51 97.505) (end 171.975 97.505) (width 0.25) (layer "F.Cu") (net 6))
 (segment (start 166.975 105.79) (end 168.225 104.54) (width 0.25) (layer "F.Cu") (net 6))
 (segment (start 164.765 103) (end 166.225 101.54) (width 0.25) (layer "F.Cu") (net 1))
 (segment (start 168.8 94.965) (end 171.975 94.965) (width 0.25) (layer "F.Cu") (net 1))
 (segment (start 162 103) (end 164.765 103) (width 0.25) (layer "F.Cu") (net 1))
 (segment (start 166.225 97.54) (end 168.8 94.965) (width 0.25) (layer "F.Cu") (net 1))
 (segment (start 166.225 101.54) (end 166.225 97.54) (width 0.25) (layer "F.Cu") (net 1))
 (segment (start 164.975 94.54) (end 167.09 92.425) (width 0.25) (layer "F.Cu") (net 2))
 (segment (start 162 94.54) (end 164.975 94.54) (width 0.25) (layer "F.Cu") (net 2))
 (segment (start 167.09 92.425) (end 171.975 92.425) (width 0.25) (layer "F.Cu") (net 2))
 (segment (start 166.975 85.04) (end 166.975 88.04) (width 0.25) (layer "F.Cu") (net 16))
 (segment (start 168.82 89.885) (end 171.975 89.885) (width 0.25) (layer "F.Cu") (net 16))
 (segment (start 165.475 83.54) (end 166.975 85.04) (width 0.25) (layer "F.Cu") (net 16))
 (segment (start 162 83.54) (end 165.475 83.54) (width 0.25) (layer "F.Cu") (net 16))
 (segment (start 166.975 88.04) (end 168.82 89.885) (width 0.25) (layer "F.Cu") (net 16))
 (segment (start 141.975 83.54) (end 152 83.54) (width 0.25) (layer "F.Cu") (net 4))
 (segment (start 141.975 81) (end 152 81) (width 0.25) (layer "F.Cu") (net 5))
 (segment (start 141.975 94.54) (end 152 94.54) (width 0.25) (layer "F.Cu") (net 8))
 (segment (start 141.975 92) (end 152 92) (width 0.25) (layer "F.Cu") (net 9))
 (segment (start 141.975 105.54) (end 152 105.54) (width 0.25) (layer "F.Cu") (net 14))
 (segment (start 141.975 103) (end 152 103) (width 0.25) (layer "F.Cu") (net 13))
 (segment (start 141.975 116.54) (end 152 116.54) (width 0.25) (layer "F.Cu") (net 11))
 (segment (start 141.975 114) (end 152 114) (width 0.25) (layer "F.Cu") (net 10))
 (segment (start 172.1 107.695) (end 172.005 107.79) (width 0.25) (layer "F.Cu") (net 29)))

